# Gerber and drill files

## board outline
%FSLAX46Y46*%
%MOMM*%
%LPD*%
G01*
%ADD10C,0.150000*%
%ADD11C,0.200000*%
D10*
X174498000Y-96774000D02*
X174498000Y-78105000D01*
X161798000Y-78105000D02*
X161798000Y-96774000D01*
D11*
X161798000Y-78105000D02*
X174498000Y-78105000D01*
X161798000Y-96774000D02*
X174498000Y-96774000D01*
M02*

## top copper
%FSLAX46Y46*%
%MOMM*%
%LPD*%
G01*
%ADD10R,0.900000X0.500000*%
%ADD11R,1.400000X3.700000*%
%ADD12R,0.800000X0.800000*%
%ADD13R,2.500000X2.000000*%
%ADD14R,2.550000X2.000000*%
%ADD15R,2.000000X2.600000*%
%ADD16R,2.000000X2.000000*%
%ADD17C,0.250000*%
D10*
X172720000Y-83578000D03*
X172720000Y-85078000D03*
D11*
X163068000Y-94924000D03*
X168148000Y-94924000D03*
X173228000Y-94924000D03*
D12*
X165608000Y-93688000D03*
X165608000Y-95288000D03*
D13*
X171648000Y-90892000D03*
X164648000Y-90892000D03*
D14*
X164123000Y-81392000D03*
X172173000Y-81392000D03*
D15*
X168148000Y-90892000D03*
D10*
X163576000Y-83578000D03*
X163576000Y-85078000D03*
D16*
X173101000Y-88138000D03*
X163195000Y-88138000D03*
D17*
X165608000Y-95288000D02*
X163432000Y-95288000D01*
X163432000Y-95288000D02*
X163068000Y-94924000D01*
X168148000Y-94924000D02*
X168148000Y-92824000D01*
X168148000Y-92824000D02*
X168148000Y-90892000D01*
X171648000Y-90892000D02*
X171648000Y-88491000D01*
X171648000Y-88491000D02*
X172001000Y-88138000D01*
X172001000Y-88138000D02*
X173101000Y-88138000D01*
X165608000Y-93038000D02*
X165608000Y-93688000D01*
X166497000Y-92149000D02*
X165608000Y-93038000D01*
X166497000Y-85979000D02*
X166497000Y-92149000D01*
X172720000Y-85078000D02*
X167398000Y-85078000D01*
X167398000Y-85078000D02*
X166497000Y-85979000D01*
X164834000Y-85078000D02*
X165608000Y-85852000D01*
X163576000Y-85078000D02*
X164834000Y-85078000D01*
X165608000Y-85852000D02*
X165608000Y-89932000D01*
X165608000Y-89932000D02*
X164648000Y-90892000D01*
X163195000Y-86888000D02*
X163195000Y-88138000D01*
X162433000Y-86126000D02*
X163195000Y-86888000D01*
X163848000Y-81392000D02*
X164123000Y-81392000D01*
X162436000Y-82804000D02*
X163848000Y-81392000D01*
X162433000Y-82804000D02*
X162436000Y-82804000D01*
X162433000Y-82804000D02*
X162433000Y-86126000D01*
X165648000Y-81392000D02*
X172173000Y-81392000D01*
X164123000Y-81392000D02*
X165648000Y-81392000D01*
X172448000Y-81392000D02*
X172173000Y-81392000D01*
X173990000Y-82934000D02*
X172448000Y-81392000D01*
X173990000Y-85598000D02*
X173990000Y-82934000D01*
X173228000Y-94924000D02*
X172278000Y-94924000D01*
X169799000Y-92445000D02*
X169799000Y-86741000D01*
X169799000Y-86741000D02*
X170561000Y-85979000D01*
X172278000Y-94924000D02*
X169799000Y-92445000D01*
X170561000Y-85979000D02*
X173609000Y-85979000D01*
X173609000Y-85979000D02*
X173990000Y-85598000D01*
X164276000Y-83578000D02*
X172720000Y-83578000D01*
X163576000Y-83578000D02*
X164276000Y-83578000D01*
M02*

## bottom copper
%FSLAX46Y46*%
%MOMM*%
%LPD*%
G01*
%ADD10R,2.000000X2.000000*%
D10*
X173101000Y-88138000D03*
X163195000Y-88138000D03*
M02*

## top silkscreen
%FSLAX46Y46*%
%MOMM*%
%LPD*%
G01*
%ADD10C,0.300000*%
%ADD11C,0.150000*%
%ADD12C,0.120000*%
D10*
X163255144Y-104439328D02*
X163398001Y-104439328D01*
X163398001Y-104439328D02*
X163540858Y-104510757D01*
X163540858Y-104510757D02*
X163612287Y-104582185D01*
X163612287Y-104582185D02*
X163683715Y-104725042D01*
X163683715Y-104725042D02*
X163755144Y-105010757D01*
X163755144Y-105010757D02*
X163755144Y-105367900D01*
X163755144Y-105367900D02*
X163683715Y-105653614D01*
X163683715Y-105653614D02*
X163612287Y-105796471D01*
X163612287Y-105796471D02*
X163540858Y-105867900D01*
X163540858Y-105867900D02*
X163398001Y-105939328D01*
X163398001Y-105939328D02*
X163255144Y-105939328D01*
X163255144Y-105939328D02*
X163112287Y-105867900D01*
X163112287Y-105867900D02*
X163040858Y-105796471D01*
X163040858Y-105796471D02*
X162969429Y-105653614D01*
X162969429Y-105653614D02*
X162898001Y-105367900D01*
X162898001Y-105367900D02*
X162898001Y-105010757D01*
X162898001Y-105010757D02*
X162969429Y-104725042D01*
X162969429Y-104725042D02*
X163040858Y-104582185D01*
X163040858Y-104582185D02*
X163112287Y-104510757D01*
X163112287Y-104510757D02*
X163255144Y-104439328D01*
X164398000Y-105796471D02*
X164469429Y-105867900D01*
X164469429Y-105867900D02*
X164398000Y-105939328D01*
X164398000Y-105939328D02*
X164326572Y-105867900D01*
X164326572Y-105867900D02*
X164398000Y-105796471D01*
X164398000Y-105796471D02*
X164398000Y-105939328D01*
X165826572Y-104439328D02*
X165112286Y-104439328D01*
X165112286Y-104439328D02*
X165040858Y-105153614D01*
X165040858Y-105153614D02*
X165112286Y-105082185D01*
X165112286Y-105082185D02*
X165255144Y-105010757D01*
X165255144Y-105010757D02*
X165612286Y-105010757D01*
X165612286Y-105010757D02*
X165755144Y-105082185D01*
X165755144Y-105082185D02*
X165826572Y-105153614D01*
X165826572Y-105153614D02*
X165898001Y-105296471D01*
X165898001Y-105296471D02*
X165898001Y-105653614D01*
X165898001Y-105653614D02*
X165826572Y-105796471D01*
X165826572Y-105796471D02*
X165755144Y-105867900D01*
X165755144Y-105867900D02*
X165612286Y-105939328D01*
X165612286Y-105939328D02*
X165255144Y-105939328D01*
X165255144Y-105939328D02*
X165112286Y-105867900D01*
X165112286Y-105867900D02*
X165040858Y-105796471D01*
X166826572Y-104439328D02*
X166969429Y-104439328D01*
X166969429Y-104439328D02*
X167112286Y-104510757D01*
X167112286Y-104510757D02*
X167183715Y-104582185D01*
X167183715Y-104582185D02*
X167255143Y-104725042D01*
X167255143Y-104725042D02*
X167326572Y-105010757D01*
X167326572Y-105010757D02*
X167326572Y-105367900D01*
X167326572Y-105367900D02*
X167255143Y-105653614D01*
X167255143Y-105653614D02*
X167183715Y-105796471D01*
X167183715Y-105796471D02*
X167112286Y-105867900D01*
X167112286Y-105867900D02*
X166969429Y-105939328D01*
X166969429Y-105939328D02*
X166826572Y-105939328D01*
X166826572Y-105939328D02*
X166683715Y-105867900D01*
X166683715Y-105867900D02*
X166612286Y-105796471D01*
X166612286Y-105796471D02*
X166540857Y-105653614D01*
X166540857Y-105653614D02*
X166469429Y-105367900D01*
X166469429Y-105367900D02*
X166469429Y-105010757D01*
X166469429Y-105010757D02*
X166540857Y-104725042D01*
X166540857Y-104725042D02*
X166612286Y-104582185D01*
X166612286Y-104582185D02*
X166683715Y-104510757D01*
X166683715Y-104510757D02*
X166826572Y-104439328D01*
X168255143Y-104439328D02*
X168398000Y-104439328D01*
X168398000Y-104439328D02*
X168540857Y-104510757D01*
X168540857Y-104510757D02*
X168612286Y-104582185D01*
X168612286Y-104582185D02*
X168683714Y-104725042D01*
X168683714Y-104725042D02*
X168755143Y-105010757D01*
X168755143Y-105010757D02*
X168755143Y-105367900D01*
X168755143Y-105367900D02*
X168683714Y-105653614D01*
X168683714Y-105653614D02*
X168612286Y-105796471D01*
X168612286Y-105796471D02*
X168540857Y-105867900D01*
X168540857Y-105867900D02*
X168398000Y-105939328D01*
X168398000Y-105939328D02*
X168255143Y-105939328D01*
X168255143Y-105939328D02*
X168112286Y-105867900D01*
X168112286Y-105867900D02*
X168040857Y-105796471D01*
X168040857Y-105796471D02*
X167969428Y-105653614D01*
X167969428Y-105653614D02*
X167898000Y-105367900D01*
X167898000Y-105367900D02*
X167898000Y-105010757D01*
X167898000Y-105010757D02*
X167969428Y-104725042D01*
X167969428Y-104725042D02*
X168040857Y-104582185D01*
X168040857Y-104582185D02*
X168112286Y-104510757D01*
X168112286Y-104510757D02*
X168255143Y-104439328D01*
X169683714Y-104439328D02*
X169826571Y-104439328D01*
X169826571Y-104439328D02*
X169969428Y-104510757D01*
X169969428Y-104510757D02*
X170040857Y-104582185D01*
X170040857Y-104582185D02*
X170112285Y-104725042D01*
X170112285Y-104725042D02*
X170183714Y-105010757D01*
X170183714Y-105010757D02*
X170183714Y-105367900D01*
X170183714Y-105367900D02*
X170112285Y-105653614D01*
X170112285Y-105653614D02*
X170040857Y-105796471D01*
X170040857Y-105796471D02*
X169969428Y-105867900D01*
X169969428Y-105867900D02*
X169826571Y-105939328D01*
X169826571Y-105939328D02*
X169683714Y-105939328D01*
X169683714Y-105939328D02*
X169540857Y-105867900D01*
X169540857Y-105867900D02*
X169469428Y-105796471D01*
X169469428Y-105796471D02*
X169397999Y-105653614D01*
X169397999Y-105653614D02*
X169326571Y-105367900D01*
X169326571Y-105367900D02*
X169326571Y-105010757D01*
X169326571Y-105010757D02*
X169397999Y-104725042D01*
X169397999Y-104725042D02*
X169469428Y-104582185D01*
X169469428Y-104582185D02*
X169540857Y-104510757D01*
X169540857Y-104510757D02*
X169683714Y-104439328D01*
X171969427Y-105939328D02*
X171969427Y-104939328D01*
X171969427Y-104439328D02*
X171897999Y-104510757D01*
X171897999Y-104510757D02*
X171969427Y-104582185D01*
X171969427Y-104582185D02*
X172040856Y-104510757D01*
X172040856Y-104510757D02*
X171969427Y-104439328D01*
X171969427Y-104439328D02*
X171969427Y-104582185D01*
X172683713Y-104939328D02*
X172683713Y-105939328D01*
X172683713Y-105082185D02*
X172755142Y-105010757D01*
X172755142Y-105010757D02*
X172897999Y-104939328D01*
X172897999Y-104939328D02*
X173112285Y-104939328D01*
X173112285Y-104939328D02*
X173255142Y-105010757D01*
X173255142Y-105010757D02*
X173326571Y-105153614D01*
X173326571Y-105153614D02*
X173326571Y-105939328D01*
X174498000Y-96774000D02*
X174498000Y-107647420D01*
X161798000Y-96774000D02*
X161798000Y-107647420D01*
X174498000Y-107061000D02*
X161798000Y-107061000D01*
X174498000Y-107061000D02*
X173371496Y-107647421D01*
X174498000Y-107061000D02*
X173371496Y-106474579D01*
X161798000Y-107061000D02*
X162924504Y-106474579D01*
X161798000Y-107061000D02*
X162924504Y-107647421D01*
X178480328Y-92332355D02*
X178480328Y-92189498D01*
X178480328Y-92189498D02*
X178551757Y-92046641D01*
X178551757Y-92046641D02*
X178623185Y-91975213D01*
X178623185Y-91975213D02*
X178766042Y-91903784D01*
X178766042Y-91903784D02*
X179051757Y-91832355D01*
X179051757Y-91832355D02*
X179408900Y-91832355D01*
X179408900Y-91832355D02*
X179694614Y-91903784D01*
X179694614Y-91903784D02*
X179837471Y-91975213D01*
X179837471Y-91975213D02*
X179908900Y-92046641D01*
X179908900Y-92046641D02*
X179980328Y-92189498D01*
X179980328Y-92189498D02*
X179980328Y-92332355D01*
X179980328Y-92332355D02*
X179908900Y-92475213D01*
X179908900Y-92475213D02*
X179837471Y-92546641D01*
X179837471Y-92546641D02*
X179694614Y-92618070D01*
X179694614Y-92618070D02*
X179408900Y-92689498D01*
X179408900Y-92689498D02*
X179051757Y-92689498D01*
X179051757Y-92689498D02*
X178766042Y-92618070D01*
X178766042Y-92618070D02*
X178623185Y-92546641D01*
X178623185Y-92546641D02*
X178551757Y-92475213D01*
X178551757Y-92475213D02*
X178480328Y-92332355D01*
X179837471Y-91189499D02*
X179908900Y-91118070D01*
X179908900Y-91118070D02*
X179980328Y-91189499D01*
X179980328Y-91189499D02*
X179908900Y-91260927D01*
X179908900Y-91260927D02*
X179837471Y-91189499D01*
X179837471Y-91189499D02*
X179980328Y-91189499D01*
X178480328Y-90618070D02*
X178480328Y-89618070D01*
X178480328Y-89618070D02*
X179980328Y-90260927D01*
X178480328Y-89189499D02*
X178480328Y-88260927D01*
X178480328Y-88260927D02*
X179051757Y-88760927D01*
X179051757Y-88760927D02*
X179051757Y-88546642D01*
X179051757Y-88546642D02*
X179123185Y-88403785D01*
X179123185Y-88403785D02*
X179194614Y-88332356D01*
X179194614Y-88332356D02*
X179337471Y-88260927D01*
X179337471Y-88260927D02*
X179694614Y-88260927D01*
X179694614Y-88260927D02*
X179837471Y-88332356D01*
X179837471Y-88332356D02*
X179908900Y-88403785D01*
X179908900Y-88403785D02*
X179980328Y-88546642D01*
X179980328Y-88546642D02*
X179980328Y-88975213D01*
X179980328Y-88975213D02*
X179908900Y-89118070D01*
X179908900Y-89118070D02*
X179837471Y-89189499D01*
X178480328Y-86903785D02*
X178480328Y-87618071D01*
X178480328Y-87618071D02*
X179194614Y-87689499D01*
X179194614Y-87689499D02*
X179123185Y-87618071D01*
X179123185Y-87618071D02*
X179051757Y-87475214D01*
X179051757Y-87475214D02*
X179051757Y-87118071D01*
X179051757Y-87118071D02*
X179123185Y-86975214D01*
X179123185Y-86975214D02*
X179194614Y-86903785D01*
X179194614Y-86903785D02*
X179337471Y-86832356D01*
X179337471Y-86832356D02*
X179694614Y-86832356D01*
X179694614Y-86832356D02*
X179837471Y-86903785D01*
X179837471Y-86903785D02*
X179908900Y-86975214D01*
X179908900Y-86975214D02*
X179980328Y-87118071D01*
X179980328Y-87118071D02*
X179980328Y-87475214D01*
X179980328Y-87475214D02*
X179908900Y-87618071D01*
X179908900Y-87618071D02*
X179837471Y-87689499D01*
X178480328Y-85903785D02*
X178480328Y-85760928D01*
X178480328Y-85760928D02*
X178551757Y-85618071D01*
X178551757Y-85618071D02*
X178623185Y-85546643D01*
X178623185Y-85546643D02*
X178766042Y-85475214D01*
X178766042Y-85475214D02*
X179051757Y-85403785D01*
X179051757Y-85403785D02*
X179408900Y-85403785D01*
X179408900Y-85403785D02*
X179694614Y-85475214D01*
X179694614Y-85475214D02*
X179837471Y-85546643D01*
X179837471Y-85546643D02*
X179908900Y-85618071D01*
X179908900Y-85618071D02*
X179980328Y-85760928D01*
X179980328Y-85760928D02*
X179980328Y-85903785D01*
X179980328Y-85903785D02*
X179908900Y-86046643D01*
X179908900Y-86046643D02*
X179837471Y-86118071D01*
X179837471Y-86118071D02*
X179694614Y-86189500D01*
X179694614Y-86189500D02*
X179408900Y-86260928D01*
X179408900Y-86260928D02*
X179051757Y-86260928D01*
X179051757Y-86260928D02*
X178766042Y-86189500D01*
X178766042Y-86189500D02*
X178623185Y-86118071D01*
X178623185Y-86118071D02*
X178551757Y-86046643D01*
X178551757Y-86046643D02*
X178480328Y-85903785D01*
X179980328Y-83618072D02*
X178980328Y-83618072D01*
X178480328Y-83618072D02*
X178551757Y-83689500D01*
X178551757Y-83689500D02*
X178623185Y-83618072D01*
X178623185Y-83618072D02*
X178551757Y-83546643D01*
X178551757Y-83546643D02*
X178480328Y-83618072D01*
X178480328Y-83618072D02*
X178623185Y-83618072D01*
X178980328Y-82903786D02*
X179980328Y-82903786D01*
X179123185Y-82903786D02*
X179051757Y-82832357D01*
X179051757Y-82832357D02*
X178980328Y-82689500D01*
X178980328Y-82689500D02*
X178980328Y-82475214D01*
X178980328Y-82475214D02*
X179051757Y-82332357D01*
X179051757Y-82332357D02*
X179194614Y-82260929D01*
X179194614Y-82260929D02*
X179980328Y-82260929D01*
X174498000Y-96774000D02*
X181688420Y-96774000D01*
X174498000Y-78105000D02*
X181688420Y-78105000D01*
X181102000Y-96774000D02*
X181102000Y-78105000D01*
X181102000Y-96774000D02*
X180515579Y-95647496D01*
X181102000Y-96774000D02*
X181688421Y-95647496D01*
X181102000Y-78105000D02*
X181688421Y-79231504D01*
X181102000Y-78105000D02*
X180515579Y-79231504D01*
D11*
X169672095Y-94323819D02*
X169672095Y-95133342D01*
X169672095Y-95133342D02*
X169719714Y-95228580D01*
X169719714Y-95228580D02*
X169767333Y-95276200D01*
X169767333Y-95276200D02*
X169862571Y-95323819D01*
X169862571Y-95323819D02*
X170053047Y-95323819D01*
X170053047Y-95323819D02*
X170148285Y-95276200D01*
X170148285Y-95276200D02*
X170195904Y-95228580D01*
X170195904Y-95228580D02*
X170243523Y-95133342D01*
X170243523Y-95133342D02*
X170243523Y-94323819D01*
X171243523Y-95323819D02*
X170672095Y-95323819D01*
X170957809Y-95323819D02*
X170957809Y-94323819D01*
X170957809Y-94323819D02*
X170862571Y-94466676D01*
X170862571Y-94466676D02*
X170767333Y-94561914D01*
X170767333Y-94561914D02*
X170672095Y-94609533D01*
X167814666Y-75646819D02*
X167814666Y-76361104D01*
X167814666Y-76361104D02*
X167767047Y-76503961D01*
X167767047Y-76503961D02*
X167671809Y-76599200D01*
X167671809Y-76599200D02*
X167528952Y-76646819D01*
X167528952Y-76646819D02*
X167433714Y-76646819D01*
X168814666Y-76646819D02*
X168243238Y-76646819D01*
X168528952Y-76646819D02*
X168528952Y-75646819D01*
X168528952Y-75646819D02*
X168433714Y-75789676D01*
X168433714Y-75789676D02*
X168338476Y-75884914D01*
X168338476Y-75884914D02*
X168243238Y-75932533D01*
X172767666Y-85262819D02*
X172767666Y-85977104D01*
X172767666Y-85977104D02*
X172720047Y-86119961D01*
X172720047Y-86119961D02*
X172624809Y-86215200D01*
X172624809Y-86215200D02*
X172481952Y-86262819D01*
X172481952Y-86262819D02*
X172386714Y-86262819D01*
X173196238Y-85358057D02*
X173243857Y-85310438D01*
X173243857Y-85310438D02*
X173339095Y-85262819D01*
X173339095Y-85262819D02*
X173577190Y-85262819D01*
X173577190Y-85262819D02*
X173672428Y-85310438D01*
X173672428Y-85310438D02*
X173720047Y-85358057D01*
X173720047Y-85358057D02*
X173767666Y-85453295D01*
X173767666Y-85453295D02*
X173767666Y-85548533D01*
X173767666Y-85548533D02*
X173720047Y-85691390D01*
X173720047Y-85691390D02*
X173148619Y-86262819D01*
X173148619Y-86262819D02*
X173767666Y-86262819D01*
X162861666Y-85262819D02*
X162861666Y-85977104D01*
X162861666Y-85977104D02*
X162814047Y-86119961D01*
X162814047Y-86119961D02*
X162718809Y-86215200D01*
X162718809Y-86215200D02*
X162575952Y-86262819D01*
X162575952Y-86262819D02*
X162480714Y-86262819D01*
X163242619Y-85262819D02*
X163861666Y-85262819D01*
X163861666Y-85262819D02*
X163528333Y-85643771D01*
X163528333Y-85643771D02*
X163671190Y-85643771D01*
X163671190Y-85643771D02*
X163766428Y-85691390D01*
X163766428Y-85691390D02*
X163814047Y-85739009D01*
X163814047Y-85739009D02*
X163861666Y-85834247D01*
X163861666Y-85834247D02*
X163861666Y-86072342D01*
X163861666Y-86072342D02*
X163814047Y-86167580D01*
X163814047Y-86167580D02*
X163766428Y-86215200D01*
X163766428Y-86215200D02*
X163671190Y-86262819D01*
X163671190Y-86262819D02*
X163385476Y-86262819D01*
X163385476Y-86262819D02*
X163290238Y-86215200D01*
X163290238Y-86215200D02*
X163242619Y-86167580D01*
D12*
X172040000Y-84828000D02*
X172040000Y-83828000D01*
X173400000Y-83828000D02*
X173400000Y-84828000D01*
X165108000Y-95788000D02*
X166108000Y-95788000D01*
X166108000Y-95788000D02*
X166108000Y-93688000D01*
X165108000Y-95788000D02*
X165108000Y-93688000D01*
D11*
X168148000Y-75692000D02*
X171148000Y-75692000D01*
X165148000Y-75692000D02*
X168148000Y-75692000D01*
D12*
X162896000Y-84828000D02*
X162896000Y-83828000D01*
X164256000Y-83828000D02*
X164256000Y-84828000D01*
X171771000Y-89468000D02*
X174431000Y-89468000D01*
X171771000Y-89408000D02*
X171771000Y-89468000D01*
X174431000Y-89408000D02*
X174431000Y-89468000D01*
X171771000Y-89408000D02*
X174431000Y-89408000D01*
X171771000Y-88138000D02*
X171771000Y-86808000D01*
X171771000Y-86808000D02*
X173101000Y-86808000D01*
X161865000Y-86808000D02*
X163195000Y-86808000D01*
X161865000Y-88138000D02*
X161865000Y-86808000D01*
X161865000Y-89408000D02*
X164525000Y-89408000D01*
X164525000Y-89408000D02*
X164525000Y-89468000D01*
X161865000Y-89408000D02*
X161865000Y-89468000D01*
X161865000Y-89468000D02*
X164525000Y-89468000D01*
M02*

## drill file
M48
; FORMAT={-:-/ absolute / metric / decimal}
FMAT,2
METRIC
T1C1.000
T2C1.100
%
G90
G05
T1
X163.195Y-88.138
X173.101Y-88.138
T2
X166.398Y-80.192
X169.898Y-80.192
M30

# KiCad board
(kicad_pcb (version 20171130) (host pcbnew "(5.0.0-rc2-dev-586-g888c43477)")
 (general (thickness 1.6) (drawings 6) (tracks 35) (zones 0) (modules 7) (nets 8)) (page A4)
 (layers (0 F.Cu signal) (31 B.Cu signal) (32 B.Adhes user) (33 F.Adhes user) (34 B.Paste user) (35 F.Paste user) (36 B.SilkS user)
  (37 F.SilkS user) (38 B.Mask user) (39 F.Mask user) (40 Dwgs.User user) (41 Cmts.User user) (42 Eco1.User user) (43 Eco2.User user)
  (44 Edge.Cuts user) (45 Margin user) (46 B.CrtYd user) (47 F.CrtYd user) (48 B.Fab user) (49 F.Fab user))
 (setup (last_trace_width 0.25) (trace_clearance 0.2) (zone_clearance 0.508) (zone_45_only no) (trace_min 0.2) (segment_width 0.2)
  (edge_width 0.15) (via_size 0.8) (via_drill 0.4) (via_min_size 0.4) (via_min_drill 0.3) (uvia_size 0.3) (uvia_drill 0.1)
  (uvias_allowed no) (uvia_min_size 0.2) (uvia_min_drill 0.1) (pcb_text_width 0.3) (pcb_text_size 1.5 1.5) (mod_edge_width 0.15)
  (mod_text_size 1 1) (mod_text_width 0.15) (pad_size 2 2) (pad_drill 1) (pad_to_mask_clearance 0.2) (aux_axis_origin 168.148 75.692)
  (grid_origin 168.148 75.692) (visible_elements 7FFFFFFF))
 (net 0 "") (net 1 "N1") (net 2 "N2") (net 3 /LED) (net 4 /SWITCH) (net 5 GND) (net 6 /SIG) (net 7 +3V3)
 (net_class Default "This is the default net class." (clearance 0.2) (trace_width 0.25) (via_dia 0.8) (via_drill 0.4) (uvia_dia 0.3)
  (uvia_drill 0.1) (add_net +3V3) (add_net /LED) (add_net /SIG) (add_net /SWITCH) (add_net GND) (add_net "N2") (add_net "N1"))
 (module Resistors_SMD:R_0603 (layer F.Cu) (at 172.72 84.328 270)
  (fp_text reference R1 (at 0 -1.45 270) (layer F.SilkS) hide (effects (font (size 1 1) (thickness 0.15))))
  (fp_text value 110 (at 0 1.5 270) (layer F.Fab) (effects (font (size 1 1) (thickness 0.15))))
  (fp_line (start 0.5 0.68) (end -0.5 0.68) (layer F.SilkS) (width 0.12))
  (fp_line (start -0.5 -0.68) (end 0.5 -0.68) (layer F.SilkS) (width 0.12))
  (pad 1 smd rect (at -0.75 0 270) (size 0.5 0.9) (layers F.Cu F.Paste F.Mask) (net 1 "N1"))
  (pad 2 smd rect (at 0.75 0 270) (size 0.5 0.9) (layers F.Cu F.Paste F.Mask) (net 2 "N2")))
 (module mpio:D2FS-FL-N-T (layer F.Cu) (at 168.148 96.774 180)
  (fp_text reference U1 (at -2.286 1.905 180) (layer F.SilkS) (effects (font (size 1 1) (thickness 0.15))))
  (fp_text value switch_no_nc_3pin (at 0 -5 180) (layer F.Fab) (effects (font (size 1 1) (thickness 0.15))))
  (pad 3 smd rect (at 5.08 1.85 180) (size 1.4 3.7) (layers F.Cu F.Paste F.Mask) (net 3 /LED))
  (pad 2 smd rect (at 0 1.85 180) (size 1.4 3.7) (layers F.Cu F.Paste F.Mask) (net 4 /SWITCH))
  (pad 1 smd rect (at -5.08 1.85 180) (size 1.4 3.7) (layers F.Cu F.Paste F.Mask) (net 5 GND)))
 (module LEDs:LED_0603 (layer F.Cu) (at 165.608 94.488 90)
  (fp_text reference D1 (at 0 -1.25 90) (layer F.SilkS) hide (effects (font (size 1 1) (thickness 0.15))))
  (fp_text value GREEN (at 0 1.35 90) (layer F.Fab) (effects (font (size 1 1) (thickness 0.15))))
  (fp_line (start -1.3 -0.5) (end -1.3 0.5) (layer F.SilkS) (width 0.12))
  (fp_line (start -1.3 0.5) (end 0.8 0.5) (layer F.SilkS) (width 0.12))
  (fp_line (start -1.3 -0.5) (end 0.8 -0.5) (layer F.SilkS) (width 0.12))
  (pad 2 smd rect (at 0.8 0 270) (size 0.8 0.8) (layers F.Cu F.Paste F.Mask) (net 2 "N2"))
  (pad 1 smd rect (at -0.8 0 270) (size 0.8 0.8) (layers F.Cu F.Paste F.Mask) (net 3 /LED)))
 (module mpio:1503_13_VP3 (layer F.Cu) (at 168.148 75.692)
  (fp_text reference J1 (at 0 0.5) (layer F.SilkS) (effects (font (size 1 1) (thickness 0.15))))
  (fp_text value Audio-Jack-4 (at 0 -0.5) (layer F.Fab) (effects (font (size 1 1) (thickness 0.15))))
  (fp_line (start 0 0) (end 3 0) (layer F.SilkS) (width 0.15))
  (fp_line (start -3 0) (end 0 0) (layer F.SilkS) (width 0.15))
  (pad "" np_thru_hole circle (at 1.75 4.5) (size 1.1 1.1) (drill 1.1) (layers *.Cu *.Mask))
  (pad "" np_thru_hole circle (at -1.75 4.5) (size 1.1 1.1) (drill 1.1) (layers *.Cu *.Mask))
  (pad 2 smd rect (at 3.5 15.2) (size 2.5 2) (layers F.Cu F.Paste F.Mask) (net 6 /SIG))
  (pad 3 smd rect (at -3.5 15.2) (size 2.5 2) (layers F.Cu F.Paste F.Mask) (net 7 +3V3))
  (pad 4 smd rect (at -4.025 5.7) (size 2.55 2) (layers F.Cu F.Paste F.Mask) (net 5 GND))
  (pad 4 smd rect (at 4.025 5.7) (size 2.55 2) (layers F.Cu F.Paste F.Mask) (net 5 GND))
  (pad 1 smd rect (at 0 15.2) (size 2 2.6) (layers F.Cu F.Paste F.Mask) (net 4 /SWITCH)))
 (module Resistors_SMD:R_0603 (layer F.Cu) (at 163.576 84.328 90)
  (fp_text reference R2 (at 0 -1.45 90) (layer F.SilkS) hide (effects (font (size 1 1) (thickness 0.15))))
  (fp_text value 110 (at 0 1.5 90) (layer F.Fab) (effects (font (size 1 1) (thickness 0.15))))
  (fp_line (start -0.5 -0.68) (end 0.5 -0.68) (layer F.SilkS) (width 0.12))
  (fp_line (start 0.5 0.68) (end -0.5 0.68) (layer F.SilkS) (width 0.12))
  (pad 2 smd rect (at 0.75 0 90) (size 0.5 0.9) (layers F.Cu F.Paste F.Mask) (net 1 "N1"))
  (pad 1 smd rect (at -0.75 0 90) (size 0.5 0.9) (layers F.Cu F.Paste F.Mask) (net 7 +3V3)))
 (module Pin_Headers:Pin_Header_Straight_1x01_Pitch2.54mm (layer F.Cu) (at 173.101 88.138)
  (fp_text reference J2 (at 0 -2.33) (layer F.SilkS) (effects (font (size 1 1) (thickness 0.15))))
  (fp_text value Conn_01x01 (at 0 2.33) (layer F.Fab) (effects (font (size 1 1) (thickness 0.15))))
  (fp_line (start -1.33 1.33) (end 1.33 1.33) (layer F.SilkS) (width 0.12))
  (fp_line (start -1.33 1.27) (end -1.33 1.33) (layer F.SilkS) (width 0.12))
  (fp_line (start 1.33 1.27) (end 1.33 1.33) (layer F.SilkS) (width 0.12))
  (fp_line (start -1.33 1.27) (end 1.33 1.27) (layer F.SilkS) (width 0.12))
  (fp_line (start -1.33 0) (end -1.33 -1.33) (layer F.SilkS) (width 0.12))
  (fp_line (start -1.33 -1.33) (end 0 -1.33) (layer F.SilkS) (width 0.12))
  (pad 1 thru_hole rect (at 0 0) (size 2 2) (drill 1) (layers *.Cu *.Mask) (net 6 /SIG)))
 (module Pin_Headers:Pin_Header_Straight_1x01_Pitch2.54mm (layer F.Cu) (at 163.195 88.138)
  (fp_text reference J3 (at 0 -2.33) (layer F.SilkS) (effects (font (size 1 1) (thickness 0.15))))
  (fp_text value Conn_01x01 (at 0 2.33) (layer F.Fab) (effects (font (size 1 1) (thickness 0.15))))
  (fp_line (start -1.33 -1.33) (end 0 -1.33) (layer F.SilkS) (width 0.12))
  (fp_line (start -1.33 0) (end -1.33 -1.33) (layer F.SilkS) (width 0.12))
  (fp_line (start -1.33 1.27) (end 1.33 1.27) (layer F.SilkS) (width 0.12))
  (fp_line (start 1.33 1.27) (end 1.33 1.33) (layer F.SilkS) (width 0.12))
  (fp_line (start -1.33 1.27) (end -1.33 1.33) (layer F.SilkS) (width 0.12))
  (fp_line (start -1.33 1.33) (end 1.33 1.33) (layer F.SilkS) (width 0.12))
  (pad 1 thru_hole rect (at 0 0) (size 2 2) (drill 1) (layers *.Cu *.Mask) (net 5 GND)))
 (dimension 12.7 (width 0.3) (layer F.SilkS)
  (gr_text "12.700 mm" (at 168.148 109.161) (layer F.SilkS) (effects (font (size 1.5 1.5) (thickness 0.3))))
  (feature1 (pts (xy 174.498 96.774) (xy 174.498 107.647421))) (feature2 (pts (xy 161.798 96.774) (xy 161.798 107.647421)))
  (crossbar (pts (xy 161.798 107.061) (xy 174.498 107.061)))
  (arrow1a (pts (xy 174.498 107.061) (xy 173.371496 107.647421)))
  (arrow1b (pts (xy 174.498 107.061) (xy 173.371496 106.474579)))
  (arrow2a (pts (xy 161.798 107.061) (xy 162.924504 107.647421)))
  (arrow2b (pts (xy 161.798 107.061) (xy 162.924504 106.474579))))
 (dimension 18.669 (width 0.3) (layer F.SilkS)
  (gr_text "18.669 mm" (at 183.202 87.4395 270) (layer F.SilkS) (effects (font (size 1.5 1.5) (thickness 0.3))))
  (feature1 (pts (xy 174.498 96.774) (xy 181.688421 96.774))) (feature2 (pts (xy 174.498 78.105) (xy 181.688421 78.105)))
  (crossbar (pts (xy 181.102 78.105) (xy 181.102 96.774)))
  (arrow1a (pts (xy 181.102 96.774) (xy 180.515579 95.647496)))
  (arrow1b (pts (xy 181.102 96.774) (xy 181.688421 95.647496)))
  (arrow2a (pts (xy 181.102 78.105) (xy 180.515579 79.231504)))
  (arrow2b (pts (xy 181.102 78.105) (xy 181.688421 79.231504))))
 (gr_line (start 174.498 96.774) (end 174.498 78.105) (layer Edge.Cuts) (width 0.15))
 (gr_line (start 161.798 78.105) (end 161.798 96.774) (layer Edge.Cuts) (width 0.15))
 (gr_line (start 161.798 78.105) (end 174.498 78.105) (layer Edge.Cuts) (width 0.2))
 (gr_line (start 161.798 96.774) (end 174.498 96.774) (layer Edge.Cuts) (width 0.2))
 (segment (start 165.608 95.288) (end 163.432 95.288) (width 0.25) (layer F.Cu) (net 3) (status 30))
 (segment (start 163.432 95.288) (end 163.068 94.924) (width 0.25) (layer F.Cu) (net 3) (status 30))
 (segment (start 168.148 94.924) (end 168.148 92.824) (width 0.25) (layer F.Cu) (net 4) (status 10))
 (segment (start 168.148 92.824) (end 168.148 90.892) (width 0.25) (layer F.Cu) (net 4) (status 20))
 (segment (start 171.648 90.892) (end 171.648 88.491) (width 0.25) (layer F.Cu) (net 6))
 (segment (start 171.648 88.491) (end 172.001 88.138) (width 0.25) (layer F.Cu) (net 6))
 (segment (start 172.001 88.138) (end 173.101 88.138) (width 0.25) (layer F.Cu) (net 6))
 (segment (start 165.608 93.038) (end 165.608 93.688) (width 0.25) (layer F.Cu) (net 2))
 (segment (start 166.497 92.149) (end 165.608 93.038) (width 0.25) (layer F.Cu) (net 2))
 (segment (start 166.497 85.979) (end 166.497 92.149) (width 0.25) (layer F.Cu) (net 2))
 (segment (start 172.72 85.078) (end 167.398 85.078) (width 0.25) (layer F.Cu) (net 2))
 (segment (start 167.398 85.078) (end 166.497 85.979) (width 0.25) (layer F.Cu) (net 2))
 (segment (start 164.834 85.078) (end 165.608 85.852) (width 0.25) (layer F.Cu) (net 7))
 (segment (start 163.576 85.078) (end 164.834 85.078) (width 0.25) (layer F.Cu) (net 7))
 (segment (start 165.608 85.852) (end 165.608 89.932) (width 0.25) (layer F.Cu) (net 7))
 (segment (start 165.608 89.932) (end 164.648 90.892) (width 0.25) (layer F.Cu) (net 7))
 (segment (start 163.195 86.888) (end 163.195 88.138) (width 0.25) (layer F.Cu) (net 5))
 (segment (start 162.433 86.126) (end 163.195 86.888) (width 0.25) (layer F.Cu) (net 5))
 (segment (start 163.848 81.392) (end 164.123 81.392) (width 0.25) (layer F.Cu) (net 5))
 (segment (start 162.436 82.804) (end 163.848 81.392) (width 0.25) (layer F.Cu) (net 5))
 (segment (start 162.433 82.804) (end 162.436 82.804) (width 0.25) (layer F.Cu) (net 5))
 (segment (start 162.433 82.804) (end 162.433 86.126) (width 0.25) (layer F.Cu) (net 5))
 (segment (start 165.648 81.392) (end 172.173 81.392) (width 0.25) (layer F.Cu) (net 5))
 (segment (start 164.123 81.392) (end 165.648 81.392) (width 0.25) (layer F.Cu) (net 5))
 (segment (start 172.448 81.392) (end 172.173 81.392) (width 0.25) (layer F.Cu) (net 5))
 (segment (start 173.99 82.934) (end 172.448 81.392) (width 0.25) (layer F.Cu) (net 5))
 (segment (start 173.99 85.598) (end 173.99 82.934) (width 0.25) (layer F.Cu) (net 5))
 (segment (start 173.228 94.924) (end 172.278 94.924) (width 0.25) (layer F.Cu) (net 5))
 (segment (start 169.799 92.445) (end 169.799 86.741) (width 0.25) (layer F.Cu) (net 5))
 (segment (start 169.799 86.741) (end 170.561 85.979) (width 0.25) (layer F.Cu) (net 5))
 (segment (start 172.278 94.924) (end 169.799 92.445) (width 0.25) (layer F.Cu) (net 5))
 (segment (start 170.561 85.979) (end 173.609 85.979) (width 0.25) (layer F.Cu) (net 5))
 (segment (start 173.609 85.979) (end 173.99 85.598) (width 0.25) (layer F.Cu) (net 5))
 (segment (start 164.276 83.578) (end 172.72 83.578) (width 0.25) (layer F.Cu) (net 1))
 (segment (start 163.576 83.578) (end 164.276 83.578) (width 0.25) (layer F.Cu) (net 1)))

